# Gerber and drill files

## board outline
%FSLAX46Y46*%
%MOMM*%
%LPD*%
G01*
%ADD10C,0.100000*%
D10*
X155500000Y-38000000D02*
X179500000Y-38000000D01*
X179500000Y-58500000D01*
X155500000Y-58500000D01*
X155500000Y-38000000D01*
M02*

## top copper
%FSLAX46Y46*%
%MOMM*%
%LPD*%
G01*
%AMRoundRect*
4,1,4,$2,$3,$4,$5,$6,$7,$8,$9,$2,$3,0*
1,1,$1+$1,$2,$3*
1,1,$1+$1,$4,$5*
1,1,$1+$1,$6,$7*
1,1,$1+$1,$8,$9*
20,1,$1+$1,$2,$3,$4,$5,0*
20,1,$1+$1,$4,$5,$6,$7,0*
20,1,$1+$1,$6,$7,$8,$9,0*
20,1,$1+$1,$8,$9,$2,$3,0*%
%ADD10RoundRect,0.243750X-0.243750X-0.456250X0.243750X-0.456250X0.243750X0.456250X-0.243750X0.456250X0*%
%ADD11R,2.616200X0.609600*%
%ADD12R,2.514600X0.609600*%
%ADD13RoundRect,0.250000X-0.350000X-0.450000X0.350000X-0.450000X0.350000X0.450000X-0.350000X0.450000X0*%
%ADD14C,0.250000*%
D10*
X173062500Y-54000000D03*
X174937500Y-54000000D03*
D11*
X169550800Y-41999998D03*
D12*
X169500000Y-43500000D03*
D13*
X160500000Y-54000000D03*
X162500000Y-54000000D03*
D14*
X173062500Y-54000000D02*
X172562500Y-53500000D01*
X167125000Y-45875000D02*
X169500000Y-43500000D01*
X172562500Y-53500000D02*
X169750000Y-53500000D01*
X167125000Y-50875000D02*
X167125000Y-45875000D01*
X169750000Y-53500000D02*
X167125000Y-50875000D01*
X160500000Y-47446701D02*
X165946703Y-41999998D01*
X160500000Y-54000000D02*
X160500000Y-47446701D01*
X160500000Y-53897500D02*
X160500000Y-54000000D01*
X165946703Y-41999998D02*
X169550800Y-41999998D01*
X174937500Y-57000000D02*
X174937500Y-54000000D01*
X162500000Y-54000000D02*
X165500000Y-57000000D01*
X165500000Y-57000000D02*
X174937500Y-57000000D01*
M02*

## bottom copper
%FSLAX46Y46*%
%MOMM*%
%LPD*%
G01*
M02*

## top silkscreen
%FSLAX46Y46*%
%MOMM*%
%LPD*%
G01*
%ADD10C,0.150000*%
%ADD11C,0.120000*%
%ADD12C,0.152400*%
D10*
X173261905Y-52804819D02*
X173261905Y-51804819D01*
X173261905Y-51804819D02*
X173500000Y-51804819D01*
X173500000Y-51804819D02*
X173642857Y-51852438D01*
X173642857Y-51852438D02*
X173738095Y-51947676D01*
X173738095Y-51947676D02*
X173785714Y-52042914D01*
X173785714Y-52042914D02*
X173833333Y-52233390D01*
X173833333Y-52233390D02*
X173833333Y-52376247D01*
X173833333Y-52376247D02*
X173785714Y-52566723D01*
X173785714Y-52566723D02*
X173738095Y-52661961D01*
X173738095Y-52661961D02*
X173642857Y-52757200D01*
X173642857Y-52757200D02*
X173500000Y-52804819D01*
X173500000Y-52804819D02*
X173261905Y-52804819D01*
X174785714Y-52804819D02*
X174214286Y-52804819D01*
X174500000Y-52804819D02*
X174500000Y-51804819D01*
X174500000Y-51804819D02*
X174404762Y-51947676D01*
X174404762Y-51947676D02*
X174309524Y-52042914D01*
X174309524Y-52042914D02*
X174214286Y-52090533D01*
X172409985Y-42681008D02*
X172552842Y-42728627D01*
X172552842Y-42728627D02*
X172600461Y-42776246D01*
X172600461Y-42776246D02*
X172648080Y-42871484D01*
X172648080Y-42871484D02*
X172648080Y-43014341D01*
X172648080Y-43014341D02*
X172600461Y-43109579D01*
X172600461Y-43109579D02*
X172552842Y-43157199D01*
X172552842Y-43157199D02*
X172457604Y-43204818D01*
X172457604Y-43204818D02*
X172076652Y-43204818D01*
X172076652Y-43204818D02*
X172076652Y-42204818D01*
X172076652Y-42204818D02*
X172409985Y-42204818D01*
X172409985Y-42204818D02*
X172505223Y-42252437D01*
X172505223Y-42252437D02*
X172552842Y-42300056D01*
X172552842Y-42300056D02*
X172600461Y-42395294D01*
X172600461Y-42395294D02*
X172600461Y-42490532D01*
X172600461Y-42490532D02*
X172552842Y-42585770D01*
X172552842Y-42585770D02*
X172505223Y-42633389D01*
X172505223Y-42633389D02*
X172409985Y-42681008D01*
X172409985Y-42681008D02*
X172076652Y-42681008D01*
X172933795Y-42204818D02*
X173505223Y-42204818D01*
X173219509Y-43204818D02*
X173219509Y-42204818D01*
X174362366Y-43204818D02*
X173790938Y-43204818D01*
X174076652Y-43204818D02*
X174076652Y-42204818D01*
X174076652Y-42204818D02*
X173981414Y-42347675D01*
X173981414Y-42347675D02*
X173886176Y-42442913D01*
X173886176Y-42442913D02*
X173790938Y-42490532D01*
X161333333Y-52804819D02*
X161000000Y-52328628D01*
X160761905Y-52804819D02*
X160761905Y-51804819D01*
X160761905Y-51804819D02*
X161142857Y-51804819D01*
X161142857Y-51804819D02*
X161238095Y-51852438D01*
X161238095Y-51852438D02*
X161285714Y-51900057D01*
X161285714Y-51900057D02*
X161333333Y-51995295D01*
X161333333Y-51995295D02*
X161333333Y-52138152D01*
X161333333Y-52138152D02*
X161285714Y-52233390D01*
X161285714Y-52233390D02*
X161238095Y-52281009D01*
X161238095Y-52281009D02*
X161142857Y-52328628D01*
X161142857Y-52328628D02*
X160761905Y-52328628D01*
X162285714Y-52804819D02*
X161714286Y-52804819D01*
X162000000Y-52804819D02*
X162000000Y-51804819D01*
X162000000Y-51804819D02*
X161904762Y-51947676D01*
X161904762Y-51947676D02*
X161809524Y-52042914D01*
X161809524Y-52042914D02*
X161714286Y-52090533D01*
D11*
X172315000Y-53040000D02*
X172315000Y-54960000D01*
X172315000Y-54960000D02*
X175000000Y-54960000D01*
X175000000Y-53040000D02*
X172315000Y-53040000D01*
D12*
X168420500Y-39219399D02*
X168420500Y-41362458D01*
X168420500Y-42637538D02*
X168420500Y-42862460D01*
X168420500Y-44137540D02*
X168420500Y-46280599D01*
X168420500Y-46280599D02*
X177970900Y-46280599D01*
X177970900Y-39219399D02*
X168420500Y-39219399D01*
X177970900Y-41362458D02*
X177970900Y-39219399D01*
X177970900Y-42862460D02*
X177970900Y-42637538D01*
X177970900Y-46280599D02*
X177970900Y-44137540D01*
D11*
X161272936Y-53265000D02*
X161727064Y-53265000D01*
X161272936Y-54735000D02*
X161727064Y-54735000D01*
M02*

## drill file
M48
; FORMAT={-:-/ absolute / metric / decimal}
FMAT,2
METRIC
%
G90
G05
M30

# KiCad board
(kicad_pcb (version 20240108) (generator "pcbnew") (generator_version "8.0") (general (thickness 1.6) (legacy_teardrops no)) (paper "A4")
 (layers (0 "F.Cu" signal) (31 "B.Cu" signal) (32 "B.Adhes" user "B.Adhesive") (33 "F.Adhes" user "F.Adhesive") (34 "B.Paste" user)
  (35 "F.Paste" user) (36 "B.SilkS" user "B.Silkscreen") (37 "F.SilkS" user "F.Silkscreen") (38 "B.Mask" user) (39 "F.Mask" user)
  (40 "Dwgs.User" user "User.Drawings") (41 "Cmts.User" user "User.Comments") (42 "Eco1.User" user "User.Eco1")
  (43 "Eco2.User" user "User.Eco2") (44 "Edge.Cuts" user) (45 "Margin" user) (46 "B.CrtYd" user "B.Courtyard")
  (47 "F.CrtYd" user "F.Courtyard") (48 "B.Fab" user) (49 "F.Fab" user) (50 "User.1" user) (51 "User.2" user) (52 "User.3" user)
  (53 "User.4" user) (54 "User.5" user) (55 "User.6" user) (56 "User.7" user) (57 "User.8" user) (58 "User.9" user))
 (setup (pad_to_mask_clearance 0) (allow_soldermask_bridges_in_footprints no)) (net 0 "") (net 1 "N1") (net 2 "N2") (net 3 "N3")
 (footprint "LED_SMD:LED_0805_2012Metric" (layer "F.Cu") (at 174 54)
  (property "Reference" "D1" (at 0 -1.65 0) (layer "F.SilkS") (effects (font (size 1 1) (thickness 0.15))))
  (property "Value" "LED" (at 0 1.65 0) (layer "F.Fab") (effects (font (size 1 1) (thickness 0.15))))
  (fp_line (start -1.685 -0.96) (end -1.685 0.96) (stroke (width 0.12) (type solid)) (layer "F.SilkS"))
  (fp_line (start -1.685 0.96) (end 1 0.96) (stroke (width 0.12) (type solid)) (layer "F.SilkS"))
  (fp_line (start 1 -0.96) (end -1.685 -0.96) (stroke (width 0.12) (type solid)) (layer "F.SilkS"))
  (pad "1" smd roundrect (at -0.9375 0) (size 0.975 1.4) (layers "F.Cu" "F.Paste" "F.Mask") (roundrect_rratio 0.25) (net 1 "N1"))
  (pad "2" smd roundrect (at 0.9375 0) (size 0.975 1.4) (layers "F.Cu" "F.Paste" "F.Mask") (roundrect_rratio 0.25) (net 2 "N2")))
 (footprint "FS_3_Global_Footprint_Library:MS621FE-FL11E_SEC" (layer "F.Cu") (at 173.1957 42.749999)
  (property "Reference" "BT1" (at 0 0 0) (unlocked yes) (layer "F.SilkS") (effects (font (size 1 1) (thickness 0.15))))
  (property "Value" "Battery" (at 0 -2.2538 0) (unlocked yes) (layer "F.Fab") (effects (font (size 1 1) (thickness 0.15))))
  (fp_line (start -4.7752 -3.5306) (end -4.7752 -1.387541) (stroke (width 0.1524) (type solid)) (layer "F.SilkS"))
  (fp_line (start -4.7752 -0.112461) (end -4.7752 0.112461) (stroke (width 0.1524) (type solid)) (layer "F.SilkS"))
  (fp_line (start -4.7752 1.387541) (end -4.7752 3.5306) (stroke (width 0.1524) (type solid)) (layer "F.SilkS"))
  (fp_line (start -4.7752 3.5306) (end 4.7752 3.5306) (stroke (width 0.1524) (type solid)) (layer "F.SilkS"))
  (fp_line (start 4.7752 -3.5306) (end -4.7752 -3.5306) (stroke (width 0.1524) (type solid)) (layer "F.SilkS"))
  (fp_line (start 4.7752 -1.387541) (end 4.7752 -3.5306) (stroke (width 0.1524) (type solid)) (layer "F.SilkS"))
  (fp_line (start 4.7752 0.112461) (end 4.7752 -0.112461) (stroke (width 0.1524) (type solid)) (layer "F.SilkS"))
  (fp_line (start 4.7752 3.5306) (end 4.7752 1.387541) (stroke (width 0.1524) (type solid)) (layer "F.SilkS"))
  (pad "1" smd rect (at -3.6449 -0.750001) (size 2.6162 0.6096) (layers "F.Cu" "F.Paste" "F.Mask") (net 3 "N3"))
  (pad "2" smd rect (at -3.6957 0.750001) (size 2.5146 0.6096) (layers "F.Cu" "F.Paste" "F.Mask") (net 1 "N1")))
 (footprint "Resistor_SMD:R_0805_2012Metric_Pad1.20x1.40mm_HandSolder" (layer "F.Cu") (at 161.5 54)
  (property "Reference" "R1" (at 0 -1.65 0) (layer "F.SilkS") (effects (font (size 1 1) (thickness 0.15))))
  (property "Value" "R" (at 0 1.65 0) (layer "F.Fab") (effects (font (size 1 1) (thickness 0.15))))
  (fp_line (start -0.227064 -0.735) (end 0.227064 -0.735) (stroke (width 0.12) (type solid)) (layer "F.SilkS"))
  (fp_line (start -0.227064 0.735) (end 0.227064 0.735) (stroke (width 0.12) (type solid)) (layer "F.SilkS"))
  (pad "1" smd roundrect (at -1 0) (size 1.2 1.4) (layers "F.Cu" "F.Paste" "F.Mask") (roundrect_rratio 0.208333) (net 3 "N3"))
  (pad "2" smd roundrect (at 1 0) (size 1.2 1.4) (layers "F.Cu" "F.Paste" "F.Mask") (roundrect_rratio 0.208333) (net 2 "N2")))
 (gr_rect (start 155.5 38) (end 179.5 58.5) (stroke (width 0.1) (type default)) (fill none) (layer "Edge.Cuts"))
 (segment (start 173.0625 54) (end 172.5625 53.5) (width 0.25) (layer "F.Cu") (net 1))
 (segment (start 167.125 45.875) (end 169.5 43.5) (width 0.25) (layer "F.Cu") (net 1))
 (segment (start 172.5625 53.5) (end 169.75 53.5) (width 0.25) (layer "F.Cu") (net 1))
 (segment (start 167.125 50.875) (end 167.125 45.875) (width 0.25) (layer "F.Cu") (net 1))
 (segment (start 169.75 53.5) (end 167.125 50.875) (width 0.25) (layer "F.Cu") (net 1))
 (segment (start 160.5 47.446701) (end 165.946703 41.999998) (width 0.25) (layer "F.Cu") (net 3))
 (segment (start 160.5 54) (end 160.5 47.446701) (width 0.25) (layer "F.Cu") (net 3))
 (segment (start 160.5 53.8975) (end 160.5 54) (width 0.25) (layer "F.Cu") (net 3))
 (segment (start 165.946703 41.999998) (end 169.5508 41.999998) (width 0.25) (layer "F.Cu") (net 3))
 (segment (start 174.9375 57) (end 174.9375 54) (width 0.25) (layer "F.Cu") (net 2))
 (segment (start 162.5 54) (end 165.5 57) (width 0.25) (layer "F.Cu") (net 2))
 (segment (start 165.5 57) (end 174.9375 57) (width 0.25) (layer "F.Cu") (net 2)))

